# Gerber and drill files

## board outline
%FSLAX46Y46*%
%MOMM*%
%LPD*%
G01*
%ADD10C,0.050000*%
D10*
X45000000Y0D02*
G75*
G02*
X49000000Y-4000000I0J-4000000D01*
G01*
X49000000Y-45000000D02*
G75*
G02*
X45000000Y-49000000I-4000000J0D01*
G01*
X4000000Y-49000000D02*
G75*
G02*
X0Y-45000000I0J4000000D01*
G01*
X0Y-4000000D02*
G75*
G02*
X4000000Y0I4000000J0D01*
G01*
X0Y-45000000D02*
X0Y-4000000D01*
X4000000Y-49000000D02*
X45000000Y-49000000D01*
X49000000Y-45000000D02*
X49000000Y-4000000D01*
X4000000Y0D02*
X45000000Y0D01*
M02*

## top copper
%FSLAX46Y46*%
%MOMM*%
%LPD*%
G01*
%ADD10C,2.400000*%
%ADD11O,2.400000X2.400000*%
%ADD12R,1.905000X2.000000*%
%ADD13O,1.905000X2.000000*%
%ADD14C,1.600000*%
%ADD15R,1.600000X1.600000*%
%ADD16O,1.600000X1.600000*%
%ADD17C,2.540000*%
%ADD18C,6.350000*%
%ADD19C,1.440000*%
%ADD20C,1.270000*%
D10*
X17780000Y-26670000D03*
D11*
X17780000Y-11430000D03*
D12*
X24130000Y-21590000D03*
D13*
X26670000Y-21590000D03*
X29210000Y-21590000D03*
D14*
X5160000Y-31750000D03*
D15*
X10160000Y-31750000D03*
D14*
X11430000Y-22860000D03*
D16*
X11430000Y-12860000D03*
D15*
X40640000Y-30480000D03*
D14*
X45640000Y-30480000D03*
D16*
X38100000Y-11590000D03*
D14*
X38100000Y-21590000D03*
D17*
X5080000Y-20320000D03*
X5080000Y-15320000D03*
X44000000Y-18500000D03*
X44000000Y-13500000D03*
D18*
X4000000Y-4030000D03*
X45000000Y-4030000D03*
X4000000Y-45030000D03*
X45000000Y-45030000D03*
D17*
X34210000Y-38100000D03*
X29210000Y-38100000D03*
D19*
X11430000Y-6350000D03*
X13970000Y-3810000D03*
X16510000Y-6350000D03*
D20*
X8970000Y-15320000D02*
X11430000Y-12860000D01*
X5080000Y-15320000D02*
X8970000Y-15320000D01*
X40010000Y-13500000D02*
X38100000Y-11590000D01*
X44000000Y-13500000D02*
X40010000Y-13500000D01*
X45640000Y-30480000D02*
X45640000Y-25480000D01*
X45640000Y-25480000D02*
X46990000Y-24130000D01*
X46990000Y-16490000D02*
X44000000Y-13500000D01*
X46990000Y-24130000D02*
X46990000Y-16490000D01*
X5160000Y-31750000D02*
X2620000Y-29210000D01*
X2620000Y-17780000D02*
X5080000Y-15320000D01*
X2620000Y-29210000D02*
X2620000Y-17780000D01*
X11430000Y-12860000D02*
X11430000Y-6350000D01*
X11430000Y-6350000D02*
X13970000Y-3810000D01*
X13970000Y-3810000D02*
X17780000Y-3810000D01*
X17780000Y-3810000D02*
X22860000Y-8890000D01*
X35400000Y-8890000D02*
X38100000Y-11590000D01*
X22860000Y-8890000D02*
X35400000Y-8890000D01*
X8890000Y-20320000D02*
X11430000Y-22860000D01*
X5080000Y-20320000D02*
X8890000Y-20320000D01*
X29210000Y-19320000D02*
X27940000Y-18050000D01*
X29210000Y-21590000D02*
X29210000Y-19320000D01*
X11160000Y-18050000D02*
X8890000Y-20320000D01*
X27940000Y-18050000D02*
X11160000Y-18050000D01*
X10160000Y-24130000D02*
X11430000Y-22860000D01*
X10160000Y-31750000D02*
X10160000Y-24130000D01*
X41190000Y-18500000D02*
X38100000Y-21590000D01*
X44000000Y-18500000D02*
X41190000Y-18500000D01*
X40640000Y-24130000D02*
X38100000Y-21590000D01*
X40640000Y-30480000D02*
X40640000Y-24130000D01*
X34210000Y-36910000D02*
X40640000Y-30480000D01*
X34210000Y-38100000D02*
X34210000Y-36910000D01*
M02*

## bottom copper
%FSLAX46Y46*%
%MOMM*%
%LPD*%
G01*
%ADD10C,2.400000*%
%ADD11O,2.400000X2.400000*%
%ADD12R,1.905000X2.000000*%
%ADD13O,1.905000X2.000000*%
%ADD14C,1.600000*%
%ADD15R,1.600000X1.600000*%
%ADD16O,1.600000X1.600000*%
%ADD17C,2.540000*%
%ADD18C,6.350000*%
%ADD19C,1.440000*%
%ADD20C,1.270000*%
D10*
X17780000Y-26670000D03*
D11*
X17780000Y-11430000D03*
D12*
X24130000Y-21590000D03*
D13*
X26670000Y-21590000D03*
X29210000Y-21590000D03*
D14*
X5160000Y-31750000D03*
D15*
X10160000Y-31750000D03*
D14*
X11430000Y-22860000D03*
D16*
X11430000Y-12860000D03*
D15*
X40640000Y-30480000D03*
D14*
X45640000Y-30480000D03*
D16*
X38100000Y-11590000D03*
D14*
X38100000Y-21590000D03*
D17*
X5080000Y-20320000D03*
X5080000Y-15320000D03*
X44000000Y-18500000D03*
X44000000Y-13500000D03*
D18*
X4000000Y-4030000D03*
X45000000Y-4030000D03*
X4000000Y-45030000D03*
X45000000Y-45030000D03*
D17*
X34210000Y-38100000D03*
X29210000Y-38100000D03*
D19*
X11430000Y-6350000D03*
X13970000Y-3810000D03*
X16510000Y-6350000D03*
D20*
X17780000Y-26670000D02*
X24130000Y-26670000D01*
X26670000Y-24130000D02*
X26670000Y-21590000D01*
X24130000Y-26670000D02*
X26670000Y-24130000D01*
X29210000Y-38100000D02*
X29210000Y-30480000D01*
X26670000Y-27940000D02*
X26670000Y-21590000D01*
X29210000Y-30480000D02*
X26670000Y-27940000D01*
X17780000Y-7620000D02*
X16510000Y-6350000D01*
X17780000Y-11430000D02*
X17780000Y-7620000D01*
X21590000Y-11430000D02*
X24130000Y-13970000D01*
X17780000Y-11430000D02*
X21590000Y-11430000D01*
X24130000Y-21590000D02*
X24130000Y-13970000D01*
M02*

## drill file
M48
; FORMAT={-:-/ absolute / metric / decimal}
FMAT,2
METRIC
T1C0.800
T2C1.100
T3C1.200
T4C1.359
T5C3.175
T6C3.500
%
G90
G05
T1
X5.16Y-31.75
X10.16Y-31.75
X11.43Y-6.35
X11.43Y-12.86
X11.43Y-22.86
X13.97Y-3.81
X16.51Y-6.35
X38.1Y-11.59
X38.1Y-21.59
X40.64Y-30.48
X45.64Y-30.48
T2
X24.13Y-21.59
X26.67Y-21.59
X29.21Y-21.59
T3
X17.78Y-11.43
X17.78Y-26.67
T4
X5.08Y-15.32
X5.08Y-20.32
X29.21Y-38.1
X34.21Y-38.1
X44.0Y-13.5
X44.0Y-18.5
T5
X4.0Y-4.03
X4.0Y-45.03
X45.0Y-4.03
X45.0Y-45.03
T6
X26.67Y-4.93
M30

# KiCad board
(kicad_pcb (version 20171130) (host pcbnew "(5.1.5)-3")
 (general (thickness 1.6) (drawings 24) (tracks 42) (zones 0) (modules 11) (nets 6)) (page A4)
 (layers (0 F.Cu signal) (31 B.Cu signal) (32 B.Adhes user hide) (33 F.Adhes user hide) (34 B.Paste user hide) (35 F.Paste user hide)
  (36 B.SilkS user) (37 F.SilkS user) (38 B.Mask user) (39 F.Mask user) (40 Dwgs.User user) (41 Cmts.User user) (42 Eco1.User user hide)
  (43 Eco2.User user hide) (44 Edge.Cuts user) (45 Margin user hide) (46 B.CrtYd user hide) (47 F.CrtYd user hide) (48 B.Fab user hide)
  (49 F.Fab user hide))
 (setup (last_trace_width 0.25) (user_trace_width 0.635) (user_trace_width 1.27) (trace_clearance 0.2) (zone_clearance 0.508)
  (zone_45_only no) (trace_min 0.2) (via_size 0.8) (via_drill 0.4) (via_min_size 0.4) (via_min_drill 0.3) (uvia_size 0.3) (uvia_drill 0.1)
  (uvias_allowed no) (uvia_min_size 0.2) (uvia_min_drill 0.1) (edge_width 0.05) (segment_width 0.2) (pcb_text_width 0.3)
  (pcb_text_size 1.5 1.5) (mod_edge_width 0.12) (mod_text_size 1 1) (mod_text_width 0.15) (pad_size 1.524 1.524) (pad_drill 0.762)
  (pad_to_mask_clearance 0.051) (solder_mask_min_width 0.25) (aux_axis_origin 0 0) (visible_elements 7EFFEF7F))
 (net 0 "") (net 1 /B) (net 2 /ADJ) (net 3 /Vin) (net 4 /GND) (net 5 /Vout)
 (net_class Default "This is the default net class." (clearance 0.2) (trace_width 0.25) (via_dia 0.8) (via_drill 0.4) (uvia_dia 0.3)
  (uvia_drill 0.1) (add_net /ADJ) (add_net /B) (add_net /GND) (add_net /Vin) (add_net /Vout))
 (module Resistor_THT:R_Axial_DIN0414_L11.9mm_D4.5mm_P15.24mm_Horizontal (layer F.Cu) (at 17.78 26.67 90)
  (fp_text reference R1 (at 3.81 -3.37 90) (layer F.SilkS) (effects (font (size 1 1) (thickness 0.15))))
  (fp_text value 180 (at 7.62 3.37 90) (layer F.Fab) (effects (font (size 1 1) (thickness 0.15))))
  (pad 1 thru_hole circle (at 0 0 90) (size 2.4 2.4) (drill 1.2) (layers *.Cu *.Mask) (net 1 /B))
  (pad 2 thru_hole oval (at 15.24 0 90) (size 2.4 2.4) (drill 1.2) (layers *.Cu *.Mask) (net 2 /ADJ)))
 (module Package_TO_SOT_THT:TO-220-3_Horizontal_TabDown (layer F.Cu) (at 24.13 21.59)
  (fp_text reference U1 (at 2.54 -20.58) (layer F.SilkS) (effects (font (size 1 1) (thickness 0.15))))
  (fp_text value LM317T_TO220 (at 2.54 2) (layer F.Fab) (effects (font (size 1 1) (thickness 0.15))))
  (pad "" np_thru_hole oval (at 2.54 -16.66) (size 3.5 3.5) (drill 3.5) (layers *.Cu *.Mask))
  (pad 1 thru_hole rect (at 0 0) (size 1.905 2) (drill 1.1) (layers *.Cu *.Mask) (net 2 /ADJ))
  (pad 2 thru_hole oval (at 2.54 0) (size 1.905 2) (drill 1.1) (layers *.Cu *.Mask) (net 1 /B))
  (pad 3 thru_hole oval (at 5.08 0) (size 1.905 2) (drill 1.1) (layers *.Cu *.Mask) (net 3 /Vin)))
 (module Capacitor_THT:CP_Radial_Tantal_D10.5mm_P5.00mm (layer F.Cu) (at 10.16 31.75 180)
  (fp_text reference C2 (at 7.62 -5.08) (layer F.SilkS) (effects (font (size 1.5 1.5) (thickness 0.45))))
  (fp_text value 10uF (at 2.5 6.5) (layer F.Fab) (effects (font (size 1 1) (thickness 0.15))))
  (pad 2 thru_hole circle (at 5 0 180) (size 1.6 1.6) (drill 0.8) (layers *.Cu *.Mask) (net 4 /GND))
  (pad 1 thru_hole rect (at 0 0 180) (size 1.6 1.6) (drill 0.8) (layers *.Cu *.Mask) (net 3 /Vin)))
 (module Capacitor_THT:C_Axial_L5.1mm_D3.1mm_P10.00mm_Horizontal (layer F.Cu) (at 11.43 22.86 90)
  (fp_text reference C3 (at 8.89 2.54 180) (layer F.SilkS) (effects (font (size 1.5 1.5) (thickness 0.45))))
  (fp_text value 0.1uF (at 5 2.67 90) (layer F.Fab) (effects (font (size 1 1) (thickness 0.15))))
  (pad 1 thru_hole circle (at 0 0 90) (size 1.6 1.6) (drill 0.8) (layers *.Cu *.Mask) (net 3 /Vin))
  (pad 2 thru_hole oval (at 10 0 90) (size 1.6 1.6) (drill 0.8) (layers *.Cu *.Mask) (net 4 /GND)))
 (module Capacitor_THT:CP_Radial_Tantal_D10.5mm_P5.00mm (layer F.Cu) (at 40.64 30.48)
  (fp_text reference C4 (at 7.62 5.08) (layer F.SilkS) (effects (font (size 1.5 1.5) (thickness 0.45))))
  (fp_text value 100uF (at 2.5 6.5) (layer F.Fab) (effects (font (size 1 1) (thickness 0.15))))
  (pad 1 thru_hole rect (at 0 0) (size 1.6 1.6) (drill 0.8) (layers *.Cu *.Mask) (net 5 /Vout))
  (pad 2 thru_hole circle (at 5 0) (size 1.6 1.6) (drill 0.8) (layers *.Cu *.Mask) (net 4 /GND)))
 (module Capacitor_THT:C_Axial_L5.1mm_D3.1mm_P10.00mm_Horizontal (layer F.Cu) (at 38.1 21.59 90)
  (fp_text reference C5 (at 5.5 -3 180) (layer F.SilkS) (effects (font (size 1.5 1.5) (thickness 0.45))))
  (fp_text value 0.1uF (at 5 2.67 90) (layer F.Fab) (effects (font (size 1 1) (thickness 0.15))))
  (pad 2 thru_hole oval (at 10 0 90) (size 1.6 1.6) (drill 0.8) (layers *.Cu *.Mask) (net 4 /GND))
  (pad 1 thru_hole circle (at 0 0 90) (size 1.6 1.6) (drill 0.8) (layers *.Cu *.Mask) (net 5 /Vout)))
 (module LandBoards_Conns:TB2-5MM (layer F.Cu) (at 5.08 20.32 90)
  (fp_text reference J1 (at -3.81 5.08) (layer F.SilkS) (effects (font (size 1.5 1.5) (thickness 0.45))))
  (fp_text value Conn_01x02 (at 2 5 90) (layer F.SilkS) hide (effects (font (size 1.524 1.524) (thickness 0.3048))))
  (pad 1 thru_hole circle (at 0 0 90) (size 2.54 2.54) (drill 1.3589) (layers *.Cu *.Mask F.SilkS) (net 3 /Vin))
  (pad 2 thru_hole circle (at 5 0 90) (size 2.54 2.54) (drill 1.3589) (layers *.Cu *.Mask F.SilkS) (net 4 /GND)))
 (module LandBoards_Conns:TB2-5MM (layer F.Cu) (at 44 13.5 270)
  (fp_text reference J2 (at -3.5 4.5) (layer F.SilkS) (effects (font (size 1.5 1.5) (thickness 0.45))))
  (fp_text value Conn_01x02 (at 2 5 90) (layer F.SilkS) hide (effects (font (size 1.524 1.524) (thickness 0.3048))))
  (pad 2 thru_hole circle (at 5 0 270) (size 2.54 2.54) (drill 1.3589) (layers *.Cu *.Mask F.SilkS) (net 5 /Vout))
  (pad 1 thru_hole circle (at 0 0 270) (size 2.54 2.54) (drill 1.3589) (layers *.Cu *.Mask F.SilkS) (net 4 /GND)))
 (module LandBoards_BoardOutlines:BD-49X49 (layer F.Cu) (at 0 49.03)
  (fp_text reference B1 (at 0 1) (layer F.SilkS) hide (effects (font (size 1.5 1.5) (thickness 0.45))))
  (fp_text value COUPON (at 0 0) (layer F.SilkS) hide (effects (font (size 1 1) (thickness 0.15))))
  (pad 1 thru_hole circle (at 4 -45) (size 6.35 6.35) (drill 3.175) (layers *.Cu *.Mask F.SilkS))
  (pad 2 thru_hole circle (at 45 -45) (size 6.35 6.35) (drill 3.175) (layers *.Cu *.Mask F.SilkS))
  (pad 3 thru_hole circle (at 4 -4) (size 6.35 6.35) (drill 3.175) (layers *.Cu *.Mask F.SilkS))
  (pad 4 thru_hole circle (at 45 -4) (size 6.35 6.35) (drill 3.175) (layers *.Cu *.Mask F.SilkS)))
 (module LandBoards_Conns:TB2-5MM (layer F.Cu) (at 29.21 38.1)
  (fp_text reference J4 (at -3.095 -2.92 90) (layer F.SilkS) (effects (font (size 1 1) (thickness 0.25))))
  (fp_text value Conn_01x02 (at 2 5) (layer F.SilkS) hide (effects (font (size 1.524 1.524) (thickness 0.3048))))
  (pad 2 thru_hole circle (at 5 0) (size 2.54 2.54) (drill 1.3589) (layers *.Cu *.Mask F.SilkS) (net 5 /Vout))
  (pad 1 thru_hole circle (at 0 0) (size 2.54 2.54) (drill 1.3589) (layers *.Cu *.Mask F.SilkS) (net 1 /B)))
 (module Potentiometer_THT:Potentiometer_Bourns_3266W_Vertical (layer F.Cu) (at 11.43 6.35 180)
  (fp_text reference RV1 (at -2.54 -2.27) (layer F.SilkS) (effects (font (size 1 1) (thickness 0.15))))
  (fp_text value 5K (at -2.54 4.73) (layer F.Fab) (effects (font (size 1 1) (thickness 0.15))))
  (pad 1 thru_hole circle (at 0 0 180) (size 1.44 1.44) (drill 0.8) (layers *.Cu *.Mask) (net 4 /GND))
  (pad 2 thru_hole circle (at -2.54 2.54 180) (size 1.44 1.44) (drill 0.8) (layers *.Cu *.Mask) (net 4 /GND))
  (pad 3 thru_hole circle (at -5.08 0 180) (size 1.44 1.44) (drill 0.8) (layers *.Cu *.Mask) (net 2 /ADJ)))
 (gr_arc (start 45 4) (end 49 4) (angle -90) (layer Edge.Cuts) (width 0.05))
 (gr_arc (start 45 45) (end 45 49) (angle -90) (layer Edge.Cuts) (width 0.05))
 (gr_arc (start 4 45) (end 0 45) (angle -90) (layer Edge.Cuts) (width 0.05))
 (gr_arc (start 4 4) (end 4 0) (angle -90) (layer Edge.Cuts) (width 0.05))
 (gr_line (start 0 45) (end 0 4) (layer Edge.Cuts) (width 0.05))
 (gr_line (start 4 49) (end 45 49) (layer Edge.Cuts) (width 0.05))
 (gr_line (start 49 45) (end 49 4) (layer Edge.Cuts) (width 0.05))
 (gr_line (start 4 0) (end 45 0) (layer Edge.Cuts) (width 0.05))
 (segment (start 8.97 15.32) (end 11.43 12.86) (width 1.27) (layer F.Cu) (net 4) (status 20))
 (segment (start 5.08 15.32) (end 8.97 15.32) (width 1.27) (layer F.Cu) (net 4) (status 10))
 (segment (start 40.01 13.5) (end 38.1 11.59) (width 1.27) (layer F.Cu) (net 4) (status 20))
 (segment (start 44 13.5) (end 40.01 13.5) (width 1.27) (layer F.Cu) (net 4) (status 10))
 (segment (start 45.64 30.48) (end 45.64 25.48) (width 1.27) (layer F.Cu) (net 4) (status 10))
 (segment (start 45.64 25.48) (end 46.99 24.13) (width 1.27) (layer F.Cu) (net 4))
 (segment (start 46.99 16.49) (end 44 13.5) (width 1.27) (layer F.Cu) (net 4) (status 20))
 (segment (start 46.99 24.13) (end 46.99 16.49) (width 1.27) (layer F.Cu) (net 4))
 (segment (start 5.16 31.75) (end 2.62 29.21) (width 1.27) (layer F.Cu) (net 4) (status 10))
 (segment (start 2.62 17.78) (end 5.08 15.32) (width 1.27) (layer F.Cu) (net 4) (status 20))
 (segment (start 2.62 29.21) (end 2.62 17.78) (width 1.27) (layer F.Cu) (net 4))
 (segment (start 11.43 12.86) (end 11.43 6.35) (width 1.27) (layer F.Cu) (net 4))
 (segment (start 11.43 6.35) (end 13.97 3.81) (width 1.27) (layer F.Cu) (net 4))
 (segment (start 13.97 3.81) (end 17.78 3.81) (width 1.27) (layer F.Cu) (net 4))
 (segment (start 17.78 3.81) (end 22.86 8.89) (width 1.27) (layer F.Cu) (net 4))
 (segment (start 35.4 8.89) (end 38.1 11.59) (width 1.27) (layer F.Cu) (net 4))
 (segment (start 22.86 8.89) (end 35.4 8.89) (width 1.27) (layer F.Cu) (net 4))
 (segment (start 8.89 20.32) (end 11.43 22.86) (width 1.27) (layer F.Cu) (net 3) (status 20))
 (segment (start 5.08 20.32) (end 8.89 20.32) (width 1.27) (layer F.Cu) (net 3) (status 10))
 (segment (start 29.21 19.32) (end 27.94 18.05) (width 1.27) (layer F.Cu) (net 3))
 (segment (start 29.21 21.59) (end 29.21 19.32) (width 1.27) (layer F.Cu) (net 3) (status 10))
 (segment (start 11.16 18.05) (end 8.89 20.32) (width 1.27) (layer F.Cu) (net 3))
 (segment (start 27.94 18.05) (end 11.16 18.05) (width 1.27) (layer F.Cu) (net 3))
 (segment (start 10.16 24.13) (end 11.43 22.86) (width 1.27) (layer F.Cu) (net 3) (status 20))
 (segment (start 10.16 31.75) (end 10.16 24.13) (width 1.27) (layer F.Cu) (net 3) (status 10))
 (segment (start 41.19 18.5) (end 38.1 21.59) (width 1.27) (layer F.Cu) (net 5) (status 20))
 (segment (start 44 18.5) (end 41.19 18.5) (width 1.27) (layer F.Cu) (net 5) (status 10))
 (segment (start 40.64 24.13) (end 38.1 21.59) (width 1.27) (layer F.Cu) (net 5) (status 20))
 (segment (start 40.64 30.48) (end 40.64 24.13) (width 1.27) (layer F.Cu) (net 5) (status 10))
 (segment (start 34.21 36.91) (end 40.64 30.48) (width 1.27) (layer F.Cu) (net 5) (status 30))
 (segment (start 34.21 38.1) (end 34.21 36.91) (width 1.27) (layer F.Cu) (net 5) (status 30))
 (segment (start 17.78 26.67) (end 24.13 26.67) (width 1.27) (layer B.Cu) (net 1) (status 10))
 (segment (start 26.67 24.13) (end 26.67 21.59) (width 1.27) (layer B.Cu) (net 1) (status 20))
 (segment (start 24.13 26.67) (end 26.67 24.13) (width 1.27) (layer B.Cu) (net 1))
 (segment (start 29.21 38.1) (end 29.21 30.48) (width 1.27) (layer B.Cu) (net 1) (status 10))
 (segment (start 26.67 27.94) (end 26.67 21.59) (width 1.27) (layer B.Cu) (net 1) (status 20))
 (segment (start 29.21 30.48) (end 26.67 27.94) (width 1.27) (layer B.Cu) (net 1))
 (segment (start 17.78 7.62) (end 16.51 6.35) (width 1.27) (layer B.Cu) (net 2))
 (segment (start 17.78 11.43) (end 17.78 7.62) (width 1.27) (layer B.Cu) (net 2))
 (segment (start 21.59 11.43) (end 24.13 13.97) (width 1.27) (layer B.Cu) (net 2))
 (segment (start 17.78 11.43) (end 21.59 11.43) (width 1.27) (layer B.Cu) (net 2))
 (segment (start 24.13 21.59) (end 24.13 13.97) (width 1.27) (layer B.Cu) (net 2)))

